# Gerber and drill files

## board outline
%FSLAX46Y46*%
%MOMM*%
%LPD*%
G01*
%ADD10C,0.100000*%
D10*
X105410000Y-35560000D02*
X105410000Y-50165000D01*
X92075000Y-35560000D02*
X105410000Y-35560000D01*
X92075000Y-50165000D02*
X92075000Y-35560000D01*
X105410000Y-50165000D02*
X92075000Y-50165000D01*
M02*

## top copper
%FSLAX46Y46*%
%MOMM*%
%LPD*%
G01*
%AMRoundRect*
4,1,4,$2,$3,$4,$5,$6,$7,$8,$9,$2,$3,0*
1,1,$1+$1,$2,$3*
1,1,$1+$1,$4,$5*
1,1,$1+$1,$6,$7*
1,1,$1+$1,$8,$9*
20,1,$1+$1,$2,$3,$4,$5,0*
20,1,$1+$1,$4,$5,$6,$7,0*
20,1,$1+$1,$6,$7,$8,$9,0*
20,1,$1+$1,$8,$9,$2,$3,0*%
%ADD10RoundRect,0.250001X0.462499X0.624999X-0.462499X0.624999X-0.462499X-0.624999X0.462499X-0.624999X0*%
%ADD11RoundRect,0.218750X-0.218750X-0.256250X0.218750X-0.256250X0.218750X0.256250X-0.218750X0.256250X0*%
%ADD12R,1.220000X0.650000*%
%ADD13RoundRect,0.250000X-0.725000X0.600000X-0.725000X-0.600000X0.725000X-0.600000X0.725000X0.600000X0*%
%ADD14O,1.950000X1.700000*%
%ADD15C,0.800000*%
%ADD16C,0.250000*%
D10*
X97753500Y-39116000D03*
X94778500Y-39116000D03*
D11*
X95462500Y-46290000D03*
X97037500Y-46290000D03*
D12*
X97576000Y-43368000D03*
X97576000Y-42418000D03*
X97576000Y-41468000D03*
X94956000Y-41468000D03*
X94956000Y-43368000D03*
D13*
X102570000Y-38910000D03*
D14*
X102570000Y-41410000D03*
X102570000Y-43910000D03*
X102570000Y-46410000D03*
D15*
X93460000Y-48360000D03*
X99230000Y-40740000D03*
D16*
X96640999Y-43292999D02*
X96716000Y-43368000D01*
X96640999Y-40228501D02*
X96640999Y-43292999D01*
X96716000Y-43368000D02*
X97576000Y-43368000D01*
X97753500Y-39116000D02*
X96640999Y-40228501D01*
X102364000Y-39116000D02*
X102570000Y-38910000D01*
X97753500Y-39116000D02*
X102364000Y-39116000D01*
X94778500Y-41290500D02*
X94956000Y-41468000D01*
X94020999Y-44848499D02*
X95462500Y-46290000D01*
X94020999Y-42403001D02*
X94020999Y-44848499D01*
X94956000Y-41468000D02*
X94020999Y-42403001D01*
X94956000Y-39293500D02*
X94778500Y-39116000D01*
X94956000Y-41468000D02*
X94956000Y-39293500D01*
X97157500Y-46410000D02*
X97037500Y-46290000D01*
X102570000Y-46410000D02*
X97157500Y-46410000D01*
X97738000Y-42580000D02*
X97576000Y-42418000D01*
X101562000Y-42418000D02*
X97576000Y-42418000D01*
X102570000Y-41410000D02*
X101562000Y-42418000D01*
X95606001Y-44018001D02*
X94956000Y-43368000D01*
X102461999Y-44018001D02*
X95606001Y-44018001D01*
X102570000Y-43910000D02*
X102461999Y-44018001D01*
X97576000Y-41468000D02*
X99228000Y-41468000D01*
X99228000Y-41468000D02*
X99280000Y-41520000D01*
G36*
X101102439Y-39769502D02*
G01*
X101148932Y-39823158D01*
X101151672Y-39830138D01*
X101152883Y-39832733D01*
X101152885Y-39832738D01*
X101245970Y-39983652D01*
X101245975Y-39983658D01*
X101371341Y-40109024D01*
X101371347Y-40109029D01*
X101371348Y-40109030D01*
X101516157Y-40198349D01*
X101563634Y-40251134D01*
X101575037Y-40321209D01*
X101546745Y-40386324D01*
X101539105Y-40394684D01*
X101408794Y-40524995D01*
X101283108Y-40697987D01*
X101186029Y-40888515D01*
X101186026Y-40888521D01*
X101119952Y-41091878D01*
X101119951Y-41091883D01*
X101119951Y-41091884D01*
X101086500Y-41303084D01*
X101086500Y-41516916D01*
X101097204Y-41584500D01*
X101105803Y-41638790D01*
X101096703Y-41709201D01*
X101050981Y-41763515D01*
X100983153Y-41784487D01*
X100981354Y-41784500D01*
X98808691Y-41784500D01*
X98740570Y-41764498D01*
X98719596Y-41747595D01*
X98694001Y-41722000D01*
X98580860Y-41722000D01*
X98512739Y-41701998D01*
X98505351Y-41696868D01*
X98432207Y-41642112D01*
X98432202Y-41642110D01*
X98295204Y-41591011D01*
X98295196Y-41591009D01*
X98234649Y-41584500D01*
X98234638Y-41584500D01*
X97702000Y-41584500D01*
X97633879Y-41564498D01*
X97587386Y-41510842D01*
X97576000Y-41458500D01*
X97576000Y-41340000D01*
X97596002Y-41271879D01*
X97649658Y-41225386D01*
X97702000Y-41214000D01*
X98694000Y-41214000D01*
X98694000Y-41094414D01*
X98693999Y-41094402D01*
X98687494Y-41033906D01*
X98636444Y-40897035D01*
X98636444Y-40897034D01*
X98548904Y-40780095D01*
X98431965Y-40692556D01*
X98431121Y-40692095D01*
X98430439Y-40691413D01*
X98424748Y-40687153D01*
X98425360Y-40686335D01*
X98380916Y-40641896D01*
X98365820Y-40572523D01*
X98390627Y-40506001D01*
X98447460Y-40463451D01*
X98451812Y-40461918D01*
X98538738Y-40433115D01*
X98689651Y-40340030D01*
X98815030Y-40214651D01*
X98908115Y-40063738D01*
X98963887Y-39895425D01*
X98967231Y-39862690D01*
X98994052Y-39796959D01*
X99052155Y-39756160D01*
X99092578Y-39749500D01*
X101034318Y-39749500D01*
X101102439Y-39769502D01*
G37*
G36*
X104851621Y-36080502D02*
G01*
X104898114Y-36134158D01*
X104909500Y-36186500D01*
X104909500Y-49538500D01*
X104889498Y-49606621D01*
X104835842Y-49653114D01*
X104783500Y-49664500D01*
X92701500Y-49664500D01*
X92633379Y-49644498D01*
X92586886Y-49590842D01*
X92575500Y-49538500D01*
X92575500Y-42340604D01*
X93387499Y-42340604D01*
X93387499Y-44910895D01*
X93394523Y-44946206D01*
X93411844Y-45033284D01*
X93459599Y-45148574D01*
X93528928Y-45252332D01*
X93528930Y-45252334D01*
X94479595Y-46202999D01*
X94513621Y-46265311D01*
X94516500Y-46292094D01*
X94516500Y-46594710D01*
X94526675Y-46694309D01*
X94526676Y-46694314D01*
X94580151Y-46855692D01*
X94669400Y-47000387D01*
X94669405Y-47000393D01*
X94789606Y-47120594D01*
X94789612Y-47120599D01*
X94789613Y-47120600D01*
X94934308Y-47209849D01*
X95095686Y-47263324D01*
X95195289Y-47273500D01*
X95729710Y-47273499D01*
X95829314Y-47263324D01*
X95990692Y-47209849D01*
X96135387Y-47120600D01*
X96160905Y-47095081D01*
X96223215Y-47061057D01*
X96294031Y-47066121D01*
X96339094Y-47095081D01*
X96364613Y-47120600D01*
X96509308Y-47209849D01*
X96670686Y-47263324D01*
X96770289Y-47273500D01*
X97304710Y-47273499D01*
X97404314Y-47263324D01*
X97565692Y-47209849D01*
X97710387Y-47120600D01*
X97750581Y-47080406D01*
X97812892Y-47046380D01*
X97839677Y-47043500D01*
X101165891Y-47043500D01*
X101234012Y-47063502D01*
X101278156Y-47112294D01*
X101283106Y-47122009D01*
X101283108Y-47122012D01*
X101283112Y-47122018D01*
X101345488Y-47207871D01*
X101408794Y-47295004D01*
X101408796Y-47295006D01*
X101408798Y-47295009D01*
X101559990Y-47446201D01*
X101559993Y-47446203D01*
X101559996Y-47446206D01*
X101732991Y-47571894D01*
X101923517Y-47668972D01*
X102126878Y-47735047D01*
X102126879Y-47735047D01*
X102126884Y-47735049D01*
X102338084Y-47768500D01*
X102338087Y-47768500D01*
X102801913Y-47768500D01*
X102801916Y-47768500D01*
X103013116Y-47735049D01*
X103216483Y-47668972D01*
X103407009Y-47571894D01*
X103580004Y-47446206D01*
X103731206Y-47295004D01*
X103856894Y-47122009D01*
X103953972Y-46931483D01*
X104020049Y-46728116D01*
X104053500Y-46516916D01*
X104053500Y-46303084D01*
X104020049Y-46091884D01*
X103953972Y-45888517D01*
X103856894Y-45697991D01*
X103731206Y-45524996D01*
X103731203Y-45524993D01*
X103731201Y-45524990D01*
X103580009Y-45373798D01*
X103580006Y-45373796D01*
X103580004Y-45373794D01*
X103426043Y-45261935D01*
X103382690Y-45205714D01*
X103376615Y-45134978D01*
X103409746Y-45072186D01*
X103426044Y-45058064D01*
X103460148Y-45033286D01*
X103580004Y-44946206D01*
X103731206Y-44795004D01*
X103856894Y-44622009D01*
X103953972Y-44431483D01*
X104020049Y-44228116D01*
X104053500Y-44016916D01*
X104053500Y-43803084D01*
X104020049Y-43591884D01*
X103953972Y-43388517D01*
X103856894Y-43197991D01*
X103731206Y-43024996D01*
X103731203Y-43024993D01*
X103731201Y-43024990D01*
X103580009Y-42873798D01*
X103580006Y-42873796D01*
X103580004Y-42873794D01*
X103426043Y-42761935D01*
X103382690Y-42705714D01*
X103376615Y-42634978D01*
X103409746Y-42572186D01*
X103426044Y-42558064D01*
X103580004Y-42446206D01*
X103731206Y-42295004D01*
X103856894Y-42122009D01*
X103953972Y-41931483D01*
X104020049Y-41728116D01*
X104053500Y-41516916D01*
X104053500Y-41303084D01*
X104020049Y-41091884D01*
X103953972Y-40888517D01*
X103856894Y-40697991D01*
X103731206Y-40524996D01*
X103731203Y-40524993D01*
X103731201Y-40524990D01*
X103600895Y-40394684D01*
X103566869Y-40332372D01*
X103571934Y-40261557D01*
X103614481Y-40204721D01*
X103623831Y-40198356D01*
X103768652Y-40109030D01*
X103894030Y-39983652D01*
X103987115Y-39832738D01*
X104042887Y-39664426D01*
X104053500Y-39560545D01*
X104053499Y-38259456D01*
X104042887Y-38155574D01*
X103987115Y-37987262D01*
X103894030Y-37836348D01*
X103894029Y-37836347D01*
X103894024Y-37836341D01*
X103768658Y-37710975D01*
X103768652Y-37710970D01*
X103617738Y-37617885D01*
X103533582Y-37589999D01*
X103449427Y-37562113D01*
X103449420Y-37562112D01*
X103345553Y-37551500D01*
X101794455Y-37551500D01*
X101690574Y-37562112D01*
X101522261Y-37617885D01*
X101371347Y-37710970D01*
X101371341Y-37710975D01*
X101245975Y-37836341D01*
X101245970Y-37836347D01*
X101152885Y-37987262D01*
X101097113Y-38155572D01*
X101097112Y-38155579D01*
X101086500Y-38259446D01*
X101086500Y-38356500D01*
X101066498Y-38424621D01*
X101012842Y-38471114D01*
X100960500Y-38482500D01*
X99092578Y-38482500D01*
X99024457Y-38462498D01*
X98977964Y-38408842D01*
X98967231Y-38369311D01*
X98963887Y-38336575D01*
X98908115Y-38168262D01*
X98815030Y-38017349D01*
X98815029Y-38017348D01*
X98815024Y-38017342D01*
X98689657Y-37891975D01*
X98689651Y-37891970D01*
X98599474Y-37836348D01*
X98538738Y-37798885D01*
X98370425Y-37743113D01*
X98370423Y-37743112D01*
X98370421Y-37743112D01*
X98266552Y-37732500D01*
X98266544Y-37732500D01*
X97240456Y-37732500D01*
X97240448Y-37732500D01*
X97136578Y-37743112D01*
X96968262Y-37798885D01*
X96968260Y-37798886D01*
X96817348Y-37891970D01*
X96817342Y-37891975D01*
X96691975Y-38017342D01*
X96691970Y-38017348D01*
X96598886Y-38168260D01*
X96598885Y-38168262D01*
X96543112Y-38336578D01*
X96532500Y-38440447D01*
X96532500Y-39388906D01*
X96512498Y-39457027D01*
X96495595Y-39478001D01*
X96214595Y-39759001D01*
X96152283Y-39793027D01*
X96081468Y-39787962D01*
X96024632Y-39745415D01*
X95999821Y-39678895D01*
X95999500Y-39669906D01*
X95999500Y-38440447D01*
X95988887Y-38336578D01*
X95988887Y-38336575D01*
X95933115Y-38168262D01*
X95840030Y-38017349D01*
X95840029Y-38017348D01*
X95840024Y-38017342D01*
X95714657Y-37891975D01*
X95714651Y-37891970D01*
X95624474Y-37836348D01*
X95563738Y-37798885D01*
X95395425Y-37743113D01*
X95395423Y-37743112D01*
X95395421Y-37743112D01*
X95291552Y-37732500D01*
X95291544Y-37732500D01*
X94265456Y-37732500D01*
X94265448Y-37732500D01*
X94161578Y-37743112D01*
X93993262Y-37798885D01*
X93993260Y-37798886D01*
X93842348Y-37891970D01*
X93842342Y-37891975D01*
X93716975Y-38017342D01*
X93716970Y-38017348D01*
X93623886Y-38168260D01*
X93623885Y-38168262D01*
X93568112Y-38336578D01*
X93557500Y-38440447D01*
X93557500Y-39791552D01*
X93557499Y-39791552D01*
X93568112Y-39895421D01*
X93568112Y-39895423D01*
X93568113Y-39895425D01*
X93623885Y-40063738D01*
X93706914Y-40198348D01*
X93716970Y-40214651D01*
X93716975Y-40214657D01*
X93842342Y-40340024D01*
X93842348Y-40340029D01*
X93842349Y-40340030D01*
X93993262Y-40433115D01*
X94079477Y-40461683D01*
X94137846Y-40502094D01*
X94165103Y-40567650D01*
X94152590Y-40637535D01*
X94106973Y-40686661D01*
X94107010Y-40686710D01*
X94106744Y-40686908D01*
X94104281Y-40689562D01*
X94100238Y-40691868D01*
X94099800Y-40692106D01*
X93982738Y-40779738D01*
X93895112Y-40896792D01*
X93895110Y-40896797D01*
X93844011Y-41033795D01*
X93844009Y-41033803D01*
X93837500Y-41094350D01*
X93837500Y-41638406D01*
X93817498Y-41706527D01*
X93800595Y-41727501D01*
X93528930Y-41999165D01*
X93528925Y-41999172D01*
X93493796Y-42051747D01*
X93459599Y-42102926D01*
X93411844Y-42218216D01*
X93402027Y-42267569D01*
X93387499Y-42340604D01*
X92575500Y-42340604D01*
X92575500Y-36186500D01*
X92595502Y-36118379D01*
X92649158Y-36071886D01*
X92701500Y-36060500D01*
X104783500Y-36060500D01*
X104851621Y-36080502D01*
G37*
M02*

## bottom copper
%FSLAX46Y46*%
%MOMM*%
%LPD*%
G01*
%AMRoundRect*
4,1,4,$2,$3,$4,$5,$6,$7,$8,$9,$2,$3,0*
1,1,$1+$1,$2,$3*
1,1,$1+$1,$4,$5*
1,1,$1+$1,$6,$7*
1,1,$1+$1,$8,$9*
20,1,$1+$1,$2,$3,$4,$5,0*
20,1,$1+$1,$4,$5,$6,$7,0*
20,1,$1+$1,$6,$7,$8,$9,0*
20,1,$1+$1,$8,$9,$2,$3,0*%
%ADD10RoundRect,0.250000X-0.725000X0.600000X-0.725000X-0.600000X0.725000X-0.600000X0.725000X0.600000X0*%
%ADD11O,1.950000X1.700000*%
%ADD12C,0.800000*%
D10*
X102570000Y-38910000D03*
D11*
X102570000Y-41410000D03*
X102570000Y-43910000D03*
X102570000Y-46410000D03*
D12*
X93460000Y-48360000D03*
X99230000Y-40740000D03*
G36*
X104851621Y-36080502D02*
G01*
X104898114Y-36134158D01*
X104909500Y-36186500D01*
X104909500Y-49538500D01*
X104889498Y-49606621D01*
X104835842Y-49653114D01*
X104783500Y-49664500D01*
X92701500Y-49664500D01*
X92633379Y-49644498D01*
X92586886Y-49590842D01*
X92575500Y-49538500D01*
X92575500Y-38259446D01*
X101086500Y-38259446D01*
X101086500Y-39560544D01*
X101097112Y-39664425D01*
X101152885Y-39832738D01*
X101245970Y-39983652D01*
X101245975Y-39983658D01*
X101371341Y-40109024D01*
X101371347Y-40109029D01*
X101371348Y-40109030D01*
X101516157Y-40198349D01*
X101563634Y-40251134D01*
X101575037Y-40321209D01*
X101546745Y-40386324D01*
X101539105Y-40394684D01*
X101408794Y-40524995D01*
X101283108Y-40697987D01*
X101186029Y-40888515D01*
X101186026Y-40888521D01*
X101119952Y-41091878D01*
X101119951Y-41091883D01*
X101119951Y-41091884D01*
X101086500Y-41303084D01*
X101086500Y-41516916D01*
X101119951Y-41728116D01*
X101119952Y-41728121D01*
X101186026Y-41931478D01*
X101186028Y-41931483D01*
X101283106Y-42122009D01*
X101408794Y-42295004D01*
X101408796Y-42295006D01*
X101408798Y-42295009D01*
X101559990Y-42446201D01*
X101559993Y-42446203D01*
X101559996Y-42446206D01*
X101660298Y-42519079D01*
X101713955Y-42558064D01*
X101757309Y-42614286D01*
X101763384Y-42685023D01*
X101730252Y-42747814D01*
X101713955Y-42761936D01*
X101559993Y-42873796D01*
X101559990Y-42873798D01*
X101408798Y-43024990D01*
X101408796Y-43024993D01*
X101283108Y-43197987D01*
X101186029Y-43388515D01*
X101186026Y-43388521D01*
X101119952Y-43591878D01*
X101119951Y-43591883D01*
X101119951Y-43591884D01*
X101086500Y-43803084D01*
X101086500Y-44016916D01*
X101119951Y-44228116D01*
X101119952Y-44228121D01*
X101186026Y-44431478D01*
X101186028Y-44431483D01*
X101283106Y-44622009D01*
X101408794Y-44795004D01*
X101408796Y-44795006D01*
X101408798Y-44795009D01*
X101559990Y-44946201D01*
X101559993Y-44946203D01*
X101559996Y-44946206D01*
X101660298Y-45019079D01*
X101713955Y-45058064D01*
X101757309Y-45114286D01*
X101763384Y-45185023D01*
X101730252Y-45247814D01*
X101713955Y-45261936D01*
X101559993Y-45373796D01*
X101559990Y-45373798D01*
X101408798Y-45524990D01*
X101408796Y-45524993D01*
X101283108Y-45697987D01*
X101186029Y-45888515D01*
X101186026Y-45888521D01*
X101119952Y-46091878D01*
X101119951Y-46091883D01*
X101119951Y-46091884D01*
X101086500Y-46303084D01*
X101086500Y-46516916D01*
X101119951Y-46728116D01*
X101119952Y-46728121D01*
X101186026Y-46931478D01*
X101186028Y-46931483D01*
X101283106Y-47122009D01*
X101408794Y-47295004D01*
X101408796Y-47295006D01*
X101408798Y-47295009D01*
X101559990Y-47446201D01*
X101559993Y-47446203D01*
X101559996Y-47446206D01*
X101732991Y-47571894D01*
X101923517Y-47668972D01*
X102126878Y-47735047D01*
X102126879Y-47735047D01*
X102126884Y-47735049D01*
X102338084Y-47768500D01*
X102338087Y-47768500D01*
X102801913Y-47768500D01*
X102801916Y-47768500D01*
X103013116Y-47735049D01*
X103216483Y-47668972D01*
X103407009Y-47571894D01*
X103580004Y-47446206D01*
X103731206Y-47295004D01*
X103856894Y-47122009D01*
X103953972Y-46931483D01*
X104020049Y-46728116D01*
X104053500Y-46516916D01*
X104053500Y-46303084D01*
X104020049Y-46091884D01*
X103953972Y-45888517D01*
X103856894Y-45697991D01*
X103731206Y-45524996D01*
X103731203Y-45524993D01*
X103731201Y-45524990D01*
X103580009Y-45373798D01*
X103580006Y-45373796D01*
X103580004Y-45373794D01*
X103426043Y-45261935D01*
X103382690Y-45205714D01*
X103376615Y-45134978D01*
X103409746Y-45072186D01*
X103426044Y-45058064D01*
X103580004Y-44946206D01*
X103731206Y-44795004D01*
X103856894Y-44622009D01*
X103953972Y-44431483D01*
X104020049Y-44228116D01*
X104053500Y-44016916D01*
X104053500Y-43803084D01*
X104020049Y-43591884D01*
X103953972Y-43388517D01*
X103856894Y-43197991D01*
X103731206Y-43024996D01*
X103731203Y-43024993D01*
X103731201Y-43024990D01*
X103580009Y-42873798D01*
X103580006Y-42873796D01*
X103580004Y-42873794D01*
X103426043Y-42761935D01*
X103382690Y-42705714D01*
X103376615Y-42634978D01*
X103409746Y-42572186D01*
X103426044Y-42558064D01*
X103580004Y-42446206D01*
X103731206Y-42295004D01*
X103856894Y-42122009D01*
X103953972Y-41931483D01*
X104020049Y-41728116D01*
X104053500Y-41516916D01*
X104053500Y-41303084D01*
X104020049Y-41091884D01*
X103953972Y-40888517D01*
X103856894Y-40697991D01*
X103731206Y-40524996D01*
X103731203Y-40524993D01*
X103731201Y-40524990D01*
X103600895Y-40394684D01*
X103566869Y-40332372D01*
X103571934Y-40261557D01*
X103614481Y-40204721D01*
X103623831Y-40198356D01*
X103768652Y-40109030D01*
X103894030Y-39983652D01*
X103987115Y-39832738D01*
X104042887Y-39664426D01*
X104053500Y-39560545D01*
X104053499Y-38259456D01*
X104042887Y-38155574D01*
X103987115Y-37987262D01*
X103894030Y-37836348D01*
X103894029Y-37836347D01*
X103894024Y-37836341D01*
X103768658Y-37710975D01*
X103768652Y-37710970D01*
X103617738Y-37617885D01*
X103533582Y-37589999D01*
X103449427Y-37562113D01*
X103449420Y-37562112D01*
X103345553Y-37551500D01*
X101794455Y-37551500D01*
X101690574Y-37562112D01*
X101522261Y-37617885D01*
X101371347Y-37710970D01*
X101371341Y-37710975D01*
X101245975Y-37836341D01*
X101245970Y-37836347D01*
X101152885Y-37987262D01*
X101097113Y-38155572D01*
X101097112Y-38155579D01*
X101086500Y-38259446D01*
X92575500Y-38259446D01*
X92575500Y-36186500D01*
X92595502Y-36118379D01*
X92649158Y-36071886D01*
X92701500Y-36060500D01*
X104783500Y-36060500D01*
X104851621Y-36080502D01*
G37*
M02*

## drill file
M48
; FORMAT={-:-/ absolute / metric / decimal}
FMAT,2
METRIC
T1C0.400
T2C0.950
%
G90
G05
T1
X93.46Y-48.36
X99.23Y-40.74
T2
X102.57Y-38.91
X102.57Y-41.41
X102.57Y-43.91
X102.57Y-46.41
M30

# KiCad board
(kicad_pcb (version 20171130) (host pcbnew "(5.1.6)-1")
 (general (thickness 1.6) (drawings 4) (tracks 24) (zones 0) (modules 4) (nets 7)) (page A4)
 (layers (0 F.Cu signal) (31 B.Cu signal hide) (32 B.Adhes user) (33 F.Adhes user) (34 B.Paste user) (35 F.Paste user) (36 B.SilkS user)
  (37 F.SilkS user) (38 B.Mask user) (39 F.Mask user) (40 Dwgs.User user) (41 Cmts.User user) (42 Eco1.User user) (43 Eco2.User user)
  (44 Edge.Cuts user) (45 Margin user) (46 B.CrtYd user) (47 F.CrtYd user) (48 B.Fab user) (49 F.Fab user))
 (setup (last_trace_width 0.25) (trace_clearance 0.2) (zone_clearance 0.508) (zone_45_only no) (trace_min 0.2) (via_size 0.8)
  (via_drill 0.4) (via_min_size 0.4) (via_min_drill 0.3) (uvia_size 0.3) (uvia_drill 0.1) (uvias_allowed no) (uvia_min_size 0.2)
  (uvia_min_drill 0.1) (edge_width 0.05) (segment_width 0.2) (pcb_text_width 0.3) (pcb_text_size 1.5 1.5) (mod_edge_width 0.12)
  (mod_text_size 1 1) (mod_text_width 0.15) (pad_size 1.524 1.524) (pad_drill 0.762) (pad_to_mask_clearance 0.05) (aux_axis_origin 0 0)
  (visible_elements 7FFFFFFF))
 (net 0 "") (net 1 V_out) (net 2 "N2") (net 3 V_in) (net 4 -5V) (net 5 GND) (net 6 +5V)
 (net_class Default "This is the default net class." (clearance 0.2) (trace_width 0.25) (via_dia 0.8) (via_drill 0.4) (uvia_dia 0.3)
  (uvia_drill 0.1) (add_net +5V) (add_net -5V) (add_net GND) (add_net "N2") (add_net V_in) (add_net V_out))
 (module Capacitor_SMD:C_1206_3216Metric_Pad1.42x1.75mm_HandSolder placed (layer F.Cu) (at 96.266 39.116 180)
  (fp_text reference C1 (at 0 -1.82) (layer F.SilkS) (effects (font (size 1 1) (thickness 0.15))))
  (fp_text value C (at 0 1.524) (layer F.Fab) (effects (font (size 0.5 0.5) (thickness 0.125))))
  (pad 1 smd roundrect (at -1.4875 0 180) (size 1.425 1.75) (layers F.Cu F.Paste F.Mask) (roundrect_rratio 0.175439) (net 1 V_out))
  (pad 2 smd roundrect (at 1.4875 0 180) (size 1.425 1.75) (layers F.Cu F.Paste F.Mask) (roundrect_rratio 0.175439) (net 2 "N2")))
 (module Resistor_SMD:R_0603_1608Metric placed (layer F.Cu) (at 96.25 46.29)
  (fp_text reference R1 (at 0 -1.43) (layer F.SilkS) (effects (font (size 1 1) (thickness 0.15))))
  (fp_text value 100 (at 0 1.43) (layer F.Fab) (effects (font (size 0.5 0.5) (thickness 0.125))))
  (pad 1 smd roundrect (at -0.7875 0) (size 0.875 0.95) (layers F.Cu F.Paste F.Mask) (roundrect_rratio 0.25) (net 2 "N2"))
  (pad 2 smd roundrect (at 0.7875 0) (size 0.875 0.95) (layers F.Cu F.Paste F.Mask) (roundrect_rratio 0.25) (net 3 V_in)))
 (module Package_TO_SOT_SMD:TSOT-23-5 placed (layer F.Cu) (at 96.266 42.418 180)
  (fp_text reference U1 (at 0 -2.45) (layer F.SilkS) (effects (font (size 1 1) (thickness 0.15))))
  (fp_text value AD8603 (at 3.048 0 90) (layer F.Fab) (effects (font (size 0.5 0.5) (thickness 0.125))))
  (pad 1 smd rect (at -1.31 -0.95 180) (size 1.22 0.65) (layers F.Cu F.Paste F.Mask) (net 1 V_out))
  (pad 2 smd rect (at -1.31 0 180) (size 1.22 0.65) (layers F.Cu F.Paste F.Mask) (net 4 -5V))
  (pad 3 smd rect (at -1.31 0.95 180) (size 1.22 0.65) (layers F.Cu F.Paste F.Mask) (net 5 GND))
  (pad 4 smd rect (at 1.31 0.95 180) (size 1.22 0.65) (layers F.Cu F.Paste F.Mask) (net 2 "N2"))
  (pad 5 smd rect (at 1.31 -0.95 180) (size 1.22 0.65) (layers F.Cu F.Paste F.Mask) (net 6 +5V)))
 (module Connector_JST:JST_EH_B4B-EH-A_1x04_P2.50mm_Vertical (layer F.Cu) (at 102.57 38.91 270)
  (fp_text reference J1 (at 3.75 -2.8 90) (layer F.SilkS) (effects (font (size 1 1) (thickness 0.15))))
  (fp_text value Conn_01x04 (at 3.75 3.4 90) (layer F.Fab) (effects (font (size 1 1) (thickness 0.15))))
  (pad 1 thru_hole roundrect (at 0 0 270) (size 1.7 1.95) (drill 0.95) (layers *.Cu *.Mask) (roundrect_rratio 0.147059) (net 1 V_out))
  (pad 2 thru_hole oval (at 2.5 0 270) (size 1.7 1.95) (drill 0.95) (layers *.Cu *.Mask) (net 4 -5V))
  (pad 3 thru_hole oval (at 5 0 270) (size 1.7 1.95) (drill 0.95) (layers *.Cu *.Mask) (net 6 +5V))
  (pad 4 thru_hole oval (at 7.5 0 270) (size 1.7 1.95) (drill 0.95) (layers *.Cu *.Mask) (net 3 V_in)))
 (gr_line (start 105.41 35.56) (end 105.41 50.165) (layer Edge.Cuts) (width 0.1))
 (gr_line (start 92.075 35.56) (end 105.41 35.56) (layer Edge.Cuts) (width 0.1))
 (gr_line (start 92.075 50.165) (end 92.075 35.56) (layer Edge.Cuts) (width 0.1))
 (gr_line (start 105.41 50.165) (end 92.075 50.165) (layer Edge.Cuts) (width 0.1))
 (segment (start 96.640999 43.292999) (end 96.716 43.368) (width 0.25) (layer F.Cu) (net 1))
 (segment (start 96.640999 40.228501) (end 96.640999 43.292999) (width 0.25) (layer F.Cu) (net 1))
 (segment (start 96.716 43.368) (end 97.576 43.368) (width 0.25) (layer F.Cu) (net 1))
 (segment (start 97.7535 39.116) (end 96.640999 40.228501) (width 0.25) (layer F.Cu) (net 1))
 (segment (start 102.364 39.116) (end 102.57 38.91) (width 0.25) (layer F.Cu) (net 1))
 (segment (start 97.7535 39.116) (end 102.364 39.116) (width 0.25) (layer F.Cu) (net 1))
 (segment (start 94.7785 41.2905) (end 94.956 41.468) (width 0.25) (layer F.Cu) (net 2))
 (segment (start 94.020999 44.848499) (end 95.4625 46.29) (width 0.25) (layer F.Cu) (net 2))
 (segment (start 94.020999 42.403001) (end 94.020999 44.848499) (width 0.25) (layer F.Cu) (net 2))
 (segment (start 94.956 41.468) (end 94.020999 42.403001) (width 0.25) (layer F.Cu) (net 2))
 (segment (start 94.956 39.2935) (end 94.7785 39.116) (width 0.25) (layer F.Cu) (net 2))
 (segment (start 94.956 41.468) (end 94.956 39.2935) (width 0.25) (layer F.Cu) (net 2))
 (segment (start 97.1575 46.41) (end 97.0375 46.29) (width 0.25) (layer F.Cu) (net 3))
 (segment (start 102.57 46.41) (end 97.1575 46.41) (width 0.25) (layer F.Cu) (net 3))
 (segment (start 97.738 42.58) (end 97.576 42.418) (width 0.25) (layer F.Cu) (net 4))
 (segment (start 101.562 42.418) (end 97.576 42.418) (width 0.25) (layer F.Cu) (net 4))
 (segment (start 102.57 41.41) (end 101.562 42.418) (width 0.25) (layer F.Cu) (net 4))
 (segment (start 95.606001 44.018001) (end 94.956 43.368) (width 0.25) (layer F.Cu) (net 6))
 (segment (start 102.461999 44.018001) (end 95.606001 44.018001) (width 0.25) (layer F.Cu) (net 6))
 (segment (start 102.57 43.91) (end 102.461999 44.018001) (width 0.25) (layer F.Cu) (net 6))
 (via (at 93.46 48.36) (size 0.8) (drill 0.4) (layers F.Cu B.Cu) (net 5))
 (via (at 99.23 40.74) (size 0.8) (drill 0.4) (layers F.Cu B.Cu) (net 5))
 (segment (start 97.576 41.468) (end 99.228 41.468) (width 0.25) (layer F.Cu) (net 5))
 (segment (start 99.228 41.468) (end 99.28 41.52) (width 0.25) (layer F.Cu) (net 5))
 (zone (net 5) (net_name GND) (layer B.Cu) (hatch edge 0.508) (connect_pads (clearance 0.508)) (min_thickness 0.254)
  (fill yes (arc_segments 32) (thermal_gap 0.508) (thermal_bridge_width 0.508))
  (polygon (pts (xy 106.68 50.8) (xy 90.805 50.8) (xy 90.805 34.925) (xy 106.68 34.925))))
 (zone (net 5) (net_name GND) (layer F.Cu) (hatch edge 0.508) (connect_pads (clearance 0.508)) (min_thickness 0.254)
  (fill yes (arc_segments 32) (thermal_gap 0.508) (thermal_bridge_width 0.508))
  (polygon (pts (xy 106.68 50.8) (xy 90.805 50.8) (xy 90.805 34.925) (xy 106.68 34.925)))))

